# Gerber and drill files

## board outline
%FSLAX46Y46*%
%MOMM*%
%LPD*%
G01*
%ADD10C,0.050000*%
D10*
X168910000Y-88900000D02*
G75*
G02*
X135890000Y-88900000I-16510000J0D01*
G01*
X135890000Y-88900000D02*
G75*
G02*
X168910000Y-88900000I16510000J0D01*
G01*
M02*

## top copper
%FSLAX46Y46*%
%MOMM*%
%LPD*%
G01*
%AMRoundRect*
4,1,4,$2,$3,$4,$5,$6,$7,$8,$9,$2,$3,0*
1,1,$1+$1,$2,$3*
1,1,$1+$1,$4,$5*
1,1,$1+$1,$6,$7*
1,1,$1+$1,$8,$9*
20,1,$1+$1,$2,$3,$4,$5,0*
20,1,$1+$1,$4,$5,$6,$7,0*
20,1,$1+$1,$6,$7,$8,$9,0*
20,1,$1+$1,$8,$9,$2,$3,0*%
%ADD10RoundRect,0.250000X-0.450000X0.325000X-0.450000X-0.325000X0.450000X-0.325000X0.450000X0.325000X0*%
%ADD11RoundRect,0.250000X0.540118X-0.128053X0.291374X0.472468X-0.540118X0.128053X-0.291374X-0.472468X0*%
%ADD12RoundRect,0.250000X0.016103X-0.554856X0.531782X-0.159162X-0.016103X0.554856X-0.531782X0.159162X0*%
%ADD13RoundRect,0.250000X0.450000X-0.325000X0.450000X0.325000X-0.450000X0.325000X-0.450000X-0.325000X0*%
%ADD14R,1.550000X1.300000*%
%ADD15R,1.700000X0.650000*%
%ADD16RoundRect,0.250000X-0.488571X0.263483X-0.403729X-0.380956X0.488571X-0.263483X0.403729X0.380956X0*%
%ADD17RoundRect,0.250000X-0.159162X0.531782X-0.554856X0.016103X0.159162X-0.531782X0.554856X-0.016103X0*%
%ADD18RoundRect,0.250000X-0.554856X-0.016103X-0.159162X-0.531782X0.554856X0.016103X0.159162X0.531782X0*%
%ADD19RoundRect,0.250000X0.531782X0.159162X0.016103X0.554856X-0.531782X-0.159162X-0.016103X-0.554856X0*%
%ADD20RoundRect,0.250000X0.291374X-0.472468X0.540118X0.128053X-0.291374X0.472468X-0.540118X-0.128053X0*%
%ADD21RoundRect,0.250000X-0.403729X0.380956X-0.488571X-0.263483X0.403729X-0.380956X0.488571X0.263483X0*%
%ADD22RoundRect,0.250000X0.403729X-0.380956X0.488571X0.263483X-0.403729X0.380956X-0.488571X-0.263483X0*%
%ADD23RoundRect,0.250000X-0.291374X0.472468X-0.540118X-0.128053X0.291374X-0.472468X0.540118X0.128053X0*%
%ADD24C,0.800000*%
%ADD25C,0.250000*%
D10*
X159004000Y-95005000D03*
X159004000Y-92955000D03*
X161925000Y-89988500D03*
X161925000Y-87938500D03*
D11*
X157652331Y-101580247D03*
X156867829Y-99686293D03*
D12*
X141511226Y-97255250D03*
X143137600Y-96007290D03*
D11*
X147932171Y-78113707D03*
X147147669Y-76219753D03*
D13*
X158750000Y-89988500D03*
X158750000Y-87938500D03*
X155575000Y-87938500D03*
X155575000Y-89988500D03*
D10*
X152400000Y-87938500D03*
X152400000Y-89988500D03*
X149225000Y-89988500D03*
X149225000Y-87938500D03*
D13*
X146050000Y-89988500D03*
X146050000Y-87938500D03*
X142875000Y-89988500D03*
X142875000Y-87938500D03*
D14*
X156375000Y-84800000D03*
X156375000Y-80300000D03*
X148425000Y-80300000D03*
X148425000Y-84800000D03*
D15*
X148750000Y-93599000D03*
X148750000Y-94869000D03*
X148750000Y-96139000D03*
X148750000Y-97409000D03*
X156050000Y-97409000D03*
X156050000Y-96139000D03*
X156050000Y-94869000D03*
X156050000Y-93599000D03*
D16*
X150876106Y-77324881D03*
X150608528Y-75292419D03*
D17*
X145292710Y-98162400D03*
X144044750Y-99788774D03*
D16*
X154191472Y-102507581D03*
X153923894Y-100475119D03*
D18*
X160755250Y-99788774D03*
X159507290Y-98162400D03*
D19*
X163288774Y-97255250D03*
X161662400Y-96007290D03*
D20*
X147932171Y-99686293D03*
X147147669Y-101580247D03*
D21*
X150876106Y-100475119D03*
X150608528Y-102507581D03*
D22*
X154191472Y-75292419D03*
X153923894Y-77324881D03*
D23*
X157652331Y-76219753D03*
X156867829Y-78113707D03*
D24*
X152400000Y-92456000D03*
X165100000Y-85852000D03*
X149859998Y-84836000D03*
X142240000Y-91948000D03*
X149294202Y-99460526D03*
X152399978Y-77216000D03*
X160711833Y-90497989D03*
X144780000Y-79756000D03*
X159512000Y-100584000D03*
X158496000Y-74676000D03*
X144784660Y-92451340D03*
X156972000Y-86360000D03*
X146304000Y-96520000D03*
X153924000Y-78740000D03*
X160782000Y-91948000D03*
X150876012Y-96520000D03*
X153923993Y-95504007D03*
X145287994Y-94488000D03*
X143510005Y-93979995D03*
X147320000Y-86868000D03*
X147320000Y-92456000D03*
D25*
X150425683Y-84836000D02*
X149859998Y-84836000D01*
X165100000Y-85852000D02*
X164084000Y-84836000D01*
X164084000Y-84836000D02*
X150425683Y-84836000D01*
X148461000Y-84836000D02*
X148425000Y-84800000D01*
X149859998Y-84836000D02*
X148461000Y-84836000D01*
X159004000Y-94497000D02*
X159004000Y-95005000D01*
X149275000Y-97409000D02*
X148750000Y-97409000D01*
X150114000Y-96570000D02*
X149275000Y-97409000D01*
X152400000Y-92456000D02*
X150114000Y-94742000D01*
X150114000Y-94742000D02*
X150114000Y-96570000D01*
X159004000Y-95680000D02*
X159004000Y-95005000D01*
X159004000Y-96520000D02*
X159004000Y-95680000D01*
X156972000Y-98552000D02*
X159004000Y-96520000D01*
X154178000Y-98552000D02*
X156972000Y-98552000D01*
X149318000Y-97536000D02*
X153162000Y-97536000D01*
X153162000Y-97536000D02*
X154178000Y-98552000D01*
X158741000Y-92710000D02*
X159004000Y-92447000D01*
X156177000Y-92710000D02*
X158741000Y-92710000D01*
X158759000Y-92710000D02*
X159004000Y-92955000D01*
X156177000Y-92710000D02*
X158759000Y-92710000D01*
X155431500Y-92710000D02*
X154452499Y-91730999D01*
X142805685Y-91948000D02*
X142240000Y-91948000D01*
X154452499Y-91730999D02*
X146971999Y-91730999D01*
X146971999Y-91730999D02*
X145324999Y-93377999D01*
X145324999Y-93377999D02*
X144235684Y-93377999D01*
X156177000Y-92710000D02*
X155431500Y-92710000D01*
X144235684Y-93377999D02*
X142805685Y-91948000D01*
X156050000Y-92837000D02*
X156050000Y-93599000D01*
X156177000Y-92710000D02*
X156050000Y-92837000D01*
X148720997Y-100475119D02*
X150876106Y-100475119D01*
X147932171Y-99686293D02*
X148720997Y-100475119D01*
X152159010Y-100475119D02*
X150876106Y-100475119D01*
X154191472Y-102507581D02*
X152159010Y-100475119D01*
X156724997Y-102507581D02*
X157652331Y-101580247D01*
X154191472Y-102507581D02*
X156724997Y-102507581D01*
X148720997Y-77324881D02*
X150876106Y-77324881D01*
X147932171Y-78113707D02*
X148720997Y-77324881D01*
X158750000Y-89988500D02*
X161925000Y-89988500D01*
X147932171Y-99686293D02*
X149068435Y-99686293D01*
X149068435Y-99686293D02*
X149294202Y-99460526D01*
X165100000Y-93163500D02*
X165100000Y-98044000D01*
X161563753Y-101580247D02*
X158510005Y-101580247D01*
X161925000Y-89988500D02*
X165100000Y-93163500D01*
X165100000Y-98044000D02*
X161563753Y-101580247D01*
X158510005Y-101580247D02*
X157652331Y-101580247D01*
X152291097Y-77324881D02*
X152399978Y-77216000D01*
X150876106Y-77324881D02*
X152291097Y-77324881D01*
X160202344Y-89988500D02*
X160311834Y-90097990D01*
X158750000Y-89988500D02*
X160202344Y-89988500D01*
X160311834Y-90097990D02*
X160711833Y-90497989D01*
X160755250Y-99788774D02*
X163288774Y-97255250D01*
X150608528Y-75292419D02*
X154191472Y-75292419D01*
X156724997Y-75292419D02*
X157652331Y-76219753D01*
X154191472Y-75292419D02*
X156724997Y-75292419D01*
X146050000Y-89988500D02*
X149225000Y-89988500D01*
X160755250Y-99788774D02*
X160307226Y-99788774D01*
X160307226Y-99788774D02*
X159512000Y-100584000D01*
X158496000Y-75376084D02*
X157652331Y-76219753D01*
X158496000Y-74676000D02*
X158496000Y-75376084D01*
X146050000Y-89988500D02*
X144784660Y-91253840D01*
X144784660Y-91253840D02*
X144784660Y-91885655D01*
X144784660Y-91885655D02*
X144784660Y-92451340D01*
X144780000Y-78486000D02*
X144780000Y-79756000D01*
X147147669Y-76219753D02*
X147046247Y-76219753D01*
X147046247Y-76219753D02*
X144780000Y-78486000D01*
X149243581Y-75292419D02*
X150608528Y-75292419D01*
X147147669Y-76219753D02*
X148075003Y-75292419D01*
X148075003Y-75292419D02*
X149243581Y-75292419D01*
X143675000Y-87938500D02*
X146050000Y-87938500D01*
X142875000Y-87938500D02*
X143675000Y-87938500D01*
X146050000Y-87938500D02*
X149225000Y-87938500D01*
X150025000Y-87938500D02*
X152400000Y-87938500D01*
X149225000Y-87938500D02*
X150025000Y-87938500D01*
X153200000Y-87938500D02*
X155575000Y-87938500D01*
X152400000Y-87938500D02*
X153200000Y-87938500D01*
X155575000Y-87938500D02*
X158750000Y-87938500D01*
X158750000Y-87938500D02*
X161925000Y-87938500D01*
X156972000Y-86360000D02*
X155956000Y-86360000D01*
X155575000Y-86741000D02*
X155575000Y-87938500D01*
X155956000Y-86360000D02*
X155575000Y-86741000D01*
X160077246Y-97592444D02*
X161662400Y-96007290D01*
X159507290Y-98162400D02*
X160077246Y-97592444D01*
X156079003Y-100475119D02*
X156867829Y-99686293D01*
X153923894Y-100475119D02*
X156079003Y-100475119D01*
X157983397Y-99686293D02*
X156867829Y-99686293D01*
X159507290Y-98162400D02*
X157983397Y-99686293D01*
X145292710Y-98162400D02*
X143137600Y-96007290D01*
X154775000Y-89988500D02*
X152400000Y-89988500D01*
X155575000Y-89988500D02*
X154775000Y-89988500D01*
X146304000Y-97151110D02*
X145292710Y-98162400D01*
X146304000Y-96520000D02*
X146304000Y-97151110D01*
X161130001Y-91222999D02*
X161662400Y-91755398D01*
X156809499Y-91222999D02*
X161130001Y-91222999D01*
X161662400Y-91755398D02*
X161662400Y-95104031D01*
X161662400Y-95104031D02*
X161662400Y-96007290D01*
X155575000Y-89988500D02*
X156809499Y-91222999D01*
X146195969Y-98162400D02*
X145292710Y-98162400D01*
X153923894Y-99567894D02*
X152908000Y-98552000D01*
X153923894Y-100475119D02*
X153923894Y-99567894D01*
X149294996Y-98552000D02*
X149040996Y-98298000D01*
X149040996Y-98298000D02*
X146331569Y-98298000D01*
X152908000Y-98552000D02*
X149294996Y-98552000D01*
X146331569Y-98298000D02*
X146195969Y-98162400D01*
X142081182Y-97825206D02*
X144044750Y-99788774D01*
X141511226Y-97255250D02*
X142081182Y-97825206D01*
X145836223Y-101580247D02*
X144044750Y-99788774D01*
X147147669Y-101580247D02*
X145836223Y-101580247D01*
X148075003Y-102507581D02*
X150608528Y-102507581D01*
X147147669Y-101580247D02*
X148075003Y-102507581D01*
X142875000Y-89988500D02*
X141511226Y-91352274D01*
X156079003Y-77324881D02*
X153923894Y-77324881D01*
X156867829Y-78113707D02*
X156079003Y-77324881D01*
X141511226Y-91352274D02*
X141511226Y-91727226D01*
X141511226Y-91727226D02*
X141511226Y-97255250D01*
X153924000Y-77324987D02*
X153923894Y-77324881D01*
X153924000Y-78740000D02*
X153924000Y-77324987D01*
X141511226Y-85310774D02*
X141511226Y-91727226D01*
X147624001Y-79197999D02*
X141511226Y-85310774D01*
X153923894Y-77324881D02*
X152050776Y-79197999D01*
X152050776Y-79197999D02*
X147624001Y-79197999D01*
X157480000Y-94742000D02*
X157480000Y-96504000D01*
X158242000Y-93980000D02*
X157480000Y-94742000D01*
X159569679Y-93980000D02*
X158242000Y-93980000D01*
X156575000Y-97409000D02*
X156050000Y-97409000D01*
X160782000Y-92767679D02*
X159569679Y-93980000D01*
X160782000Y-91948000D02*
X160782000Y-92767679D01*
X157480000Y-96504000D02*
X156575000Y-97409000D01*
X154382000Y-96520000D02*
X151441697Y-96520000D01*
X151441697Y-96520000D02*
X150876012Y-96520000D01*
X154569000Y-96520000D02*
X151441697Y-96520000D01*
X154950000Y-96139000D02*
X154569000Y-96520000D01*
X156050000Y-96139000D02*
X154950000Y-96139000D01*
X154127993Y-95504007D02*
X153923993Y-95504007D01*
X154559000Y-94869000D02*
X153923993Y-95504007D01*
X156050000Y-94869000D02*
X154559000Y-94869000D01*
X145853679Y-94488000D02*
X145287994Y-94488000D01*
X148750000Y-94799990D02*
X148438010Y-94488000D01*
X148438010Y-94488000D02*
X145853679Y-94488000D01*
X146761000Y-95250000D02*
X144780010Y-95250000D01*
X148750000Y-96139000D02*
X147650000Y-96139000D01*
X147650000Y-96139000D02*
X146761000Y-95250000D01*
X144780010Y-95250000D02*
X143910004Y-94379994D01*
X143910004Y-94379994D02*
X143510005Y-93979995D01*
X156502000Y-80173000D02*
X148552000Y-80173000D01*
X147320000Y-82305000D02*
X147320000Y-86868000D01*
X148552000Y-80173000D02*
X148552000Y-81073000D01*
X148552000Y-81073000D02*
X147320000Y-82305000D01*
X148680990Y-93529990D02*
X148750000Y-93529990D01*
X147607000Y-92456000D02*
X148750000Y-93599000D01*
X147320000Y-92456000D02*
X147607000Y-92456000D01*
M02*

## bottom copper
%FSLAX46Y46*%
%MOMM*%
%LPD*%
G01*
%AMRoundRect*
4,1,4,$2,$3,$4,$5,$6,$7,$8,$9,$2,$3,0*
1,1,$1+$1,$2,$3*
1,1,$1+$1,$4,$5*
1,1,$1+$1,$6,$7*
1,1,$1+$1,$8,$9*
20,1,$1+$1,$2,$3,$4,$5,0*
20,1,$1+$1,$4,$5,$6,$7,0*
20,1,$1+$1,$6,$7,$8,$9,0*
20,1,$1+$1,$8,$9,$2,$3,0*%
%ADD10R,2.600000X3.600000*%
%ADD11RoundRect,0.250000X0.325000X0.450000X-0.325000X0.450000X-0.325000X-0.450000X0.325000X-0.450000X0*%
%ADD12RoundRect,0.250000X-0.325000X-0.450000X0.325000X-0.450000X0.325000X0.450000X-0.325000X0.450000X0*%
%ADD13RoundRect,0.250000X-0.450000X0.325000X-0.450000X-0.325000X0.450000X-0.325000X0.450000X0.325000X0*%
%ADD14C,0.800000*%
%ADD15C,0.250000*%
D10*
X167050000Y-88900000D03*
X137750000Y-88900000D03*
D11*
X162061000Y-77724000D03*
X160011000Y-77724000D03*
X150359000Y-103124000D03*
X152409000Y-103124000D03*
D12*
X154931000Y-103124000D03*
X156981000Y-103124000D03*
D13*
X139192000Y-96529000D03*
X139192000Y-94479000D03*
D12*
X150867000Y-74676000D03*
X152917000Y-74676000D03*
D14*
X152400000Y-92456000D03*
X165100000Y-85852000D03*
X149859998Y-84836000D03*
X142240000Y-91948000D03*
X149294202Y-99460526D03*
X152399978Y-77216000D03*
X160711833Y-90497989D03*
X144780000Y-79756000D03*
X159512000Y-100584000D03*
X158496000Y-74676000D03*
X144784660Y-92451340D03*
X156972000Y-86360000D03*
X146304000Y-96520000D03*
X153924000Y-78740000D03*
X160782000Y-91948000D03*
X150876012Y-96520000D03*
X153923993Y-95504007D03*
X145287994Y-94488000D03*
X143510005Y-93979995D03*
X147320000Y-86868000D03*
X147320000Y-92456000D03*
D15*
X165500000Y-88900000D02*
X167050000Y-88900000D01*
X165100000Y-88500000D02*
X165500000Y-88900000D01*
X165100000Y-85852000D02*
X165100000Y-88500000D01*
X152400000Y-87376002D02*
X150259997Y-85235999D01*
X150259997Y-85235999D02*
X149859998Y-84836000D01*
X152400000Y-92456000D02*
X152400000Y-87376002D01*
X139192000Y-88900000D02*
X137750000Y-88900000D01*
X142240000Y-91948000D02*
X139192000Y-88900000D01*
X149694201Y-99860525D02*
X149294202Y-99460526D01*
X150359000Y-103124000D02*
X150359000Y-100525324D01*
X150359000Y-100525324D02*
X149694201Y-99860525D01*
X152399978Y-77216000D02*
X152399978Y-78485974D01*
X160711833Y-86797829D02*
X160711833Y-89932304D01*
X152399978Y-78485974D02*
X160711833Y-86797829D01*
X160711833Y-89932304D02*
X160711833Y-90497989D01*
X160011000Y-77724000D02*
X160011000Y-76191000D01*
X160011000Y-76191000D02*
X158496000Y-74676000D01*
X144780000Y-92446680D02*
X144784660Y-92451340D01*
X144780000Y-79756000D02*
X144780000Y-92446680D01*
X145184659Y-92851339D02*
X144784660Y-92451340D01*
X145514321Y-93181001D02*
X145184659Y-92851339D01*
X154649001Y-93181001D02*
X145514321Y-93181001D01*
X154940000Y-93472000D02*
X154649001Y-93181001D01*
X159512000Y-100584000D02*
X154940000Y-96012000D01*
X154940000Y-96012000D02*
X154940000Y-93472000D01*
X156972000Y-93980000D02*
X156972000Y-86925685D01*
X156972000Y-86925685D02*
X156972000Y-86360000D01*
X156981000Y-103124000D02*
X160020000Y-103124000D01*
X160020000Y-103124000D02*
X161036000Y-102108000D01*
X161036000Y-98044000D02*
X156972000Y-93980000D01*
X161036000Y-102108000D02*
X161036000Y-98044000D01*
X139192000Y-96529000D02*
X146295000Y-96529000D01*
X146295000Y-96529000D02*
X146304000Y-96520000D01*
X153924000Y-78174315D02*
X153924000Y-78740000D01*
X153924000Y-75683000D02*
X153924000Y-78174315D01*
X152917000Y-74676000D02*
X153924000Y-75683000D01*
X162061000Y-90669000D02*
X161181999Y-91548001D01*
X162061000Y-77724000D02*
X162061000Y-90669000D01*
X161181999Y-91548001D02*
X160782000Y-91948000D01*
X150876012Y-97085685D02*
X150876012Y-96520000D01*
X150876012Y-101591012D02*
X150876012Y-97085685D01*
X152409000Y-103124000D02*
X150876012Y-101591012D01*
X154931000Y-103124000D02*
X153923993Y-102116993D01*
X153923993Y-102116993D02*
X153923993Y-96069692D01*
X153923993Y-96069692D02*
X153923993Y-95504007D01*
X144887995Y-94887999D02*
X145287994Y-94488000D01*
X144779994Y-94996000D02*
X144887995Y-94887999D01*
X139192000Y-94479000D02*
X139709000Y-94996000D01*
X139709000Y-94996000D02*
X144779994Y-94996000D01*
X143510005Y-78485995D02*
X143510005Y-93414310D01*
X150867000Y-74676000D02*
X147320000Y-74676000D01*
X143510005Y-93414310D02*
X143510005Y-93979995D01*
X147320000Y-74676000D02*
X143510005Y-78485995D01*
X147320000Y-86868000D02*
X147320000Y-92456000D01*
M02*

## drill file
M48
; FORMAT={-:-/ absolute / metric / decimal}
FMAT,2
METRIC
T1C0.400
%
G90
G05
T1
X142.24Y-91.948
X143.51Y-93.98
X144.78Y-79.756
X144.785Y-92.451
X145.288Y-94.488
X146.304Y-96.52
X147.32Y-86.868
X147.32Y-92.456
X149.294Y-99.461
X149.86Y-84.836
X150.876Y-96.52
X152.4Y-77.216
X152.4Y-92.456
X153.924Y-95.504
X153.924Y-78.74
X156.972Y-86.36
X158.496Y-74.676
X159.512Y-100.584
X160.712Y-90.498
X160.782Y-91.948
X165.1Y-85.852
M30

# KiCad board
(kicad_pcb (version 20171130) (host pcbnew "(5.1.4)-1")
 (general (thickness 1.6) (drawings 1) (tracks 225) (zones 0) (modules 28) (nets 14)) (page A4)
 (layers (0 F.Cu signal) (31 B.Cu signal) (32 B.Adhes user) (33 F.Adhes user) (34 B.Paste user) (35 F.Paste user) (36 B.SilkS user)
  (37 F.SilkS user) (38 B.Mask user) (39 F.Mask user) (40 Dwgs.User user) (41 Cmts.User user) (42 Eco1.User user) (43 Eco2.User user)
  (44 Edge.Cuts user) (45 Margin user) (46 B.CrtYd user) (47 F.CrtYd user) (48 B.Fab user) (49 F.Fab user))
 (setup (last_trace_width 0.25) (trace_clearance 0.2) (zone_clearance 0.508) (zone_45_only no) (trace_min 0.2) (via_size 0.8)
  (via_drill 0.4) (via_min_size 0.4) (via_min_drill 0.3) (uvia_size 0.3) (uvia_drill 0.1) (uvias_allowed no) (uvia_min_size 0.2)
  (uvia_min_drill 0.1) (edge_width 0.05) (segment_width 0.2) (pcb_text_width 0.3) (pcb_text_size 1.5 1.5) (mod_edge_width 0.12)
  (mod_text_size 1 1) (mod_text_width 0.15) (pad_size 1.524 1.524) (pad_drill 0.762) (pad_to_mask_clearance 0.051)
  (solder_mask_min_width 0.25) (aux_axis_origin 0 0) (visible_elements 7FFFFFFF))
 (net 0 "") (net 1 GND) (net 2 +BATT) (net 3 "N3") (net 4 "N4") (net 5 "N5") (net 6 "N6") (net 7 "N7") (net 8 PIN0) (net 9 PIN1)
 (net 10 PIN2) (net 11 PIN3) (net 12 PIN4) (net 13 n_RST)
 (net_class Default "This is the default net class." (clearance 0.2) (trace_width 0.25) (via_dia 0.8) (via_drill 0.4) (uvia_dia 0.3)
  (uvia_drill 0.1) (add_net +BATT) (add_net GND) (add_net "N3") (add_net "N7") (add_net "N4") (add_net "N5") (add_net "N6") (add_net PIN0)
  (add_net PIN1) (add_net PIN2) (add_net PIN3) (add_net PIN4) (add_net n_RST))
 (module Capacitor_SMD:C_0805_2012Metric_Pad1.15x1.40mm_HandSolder (layer F.Cu) (at 159.004 93.98 270)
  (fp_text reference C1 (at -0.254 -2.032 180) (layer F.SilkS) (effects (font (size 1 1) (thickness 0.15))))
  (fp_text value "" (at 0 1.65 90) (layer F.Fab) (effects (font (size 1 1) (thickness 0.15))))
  (pad 2 smd roundrect (at 1.025 0 270) (size 1.15 1.4) (layers F.Cu F.Paste F.Mask) (roundrect_rratio 0.217391) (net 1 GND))
  (pad 1 smd roundrect (at -1.025 0 270) (size 1.15 1.4) (layers F.Cu F.Paste F.Mask) (roundrect_rratio 0.217391) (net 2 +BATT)))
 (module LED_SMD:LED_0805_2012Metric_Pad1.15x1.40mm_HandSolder (layer F.Cu) (at 161.925 88.9635 270)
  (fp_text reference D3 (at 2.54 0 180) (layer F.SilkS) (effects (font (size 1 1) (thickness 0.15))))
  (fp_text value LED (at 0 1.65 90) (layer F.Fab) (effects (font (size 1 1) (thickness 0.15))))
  (pad 2 smd roundrect (at 1.025 0 270) (size 1.15 1.4) (layers F.Cu F.Paste F.Mask) (roundrect_rratio 0.217391) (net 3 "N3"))
  (pad 1 smd roundrect (at -1.025 0 270) (size 1.15 1.4) (layers F.Cu F.Paste F.Mask) (roundrect_rratio 0.217391) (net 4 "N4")))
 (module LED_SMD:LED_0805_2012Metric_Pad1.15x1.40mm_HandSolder (layer F.Cu) (at 157.26008 100.63327 112.5)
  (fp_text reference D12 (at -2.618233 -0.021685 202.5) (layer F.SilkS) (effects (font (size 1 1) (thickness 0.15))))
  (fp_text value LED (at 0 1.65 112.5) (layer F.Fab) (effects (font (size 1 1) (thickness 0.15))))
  (pad 1 smd roundrect (at -1.025 0 112.5) (size 1.15 1.4) (layers F.Cu F.Paste F.Mask) (roundrect_rratio 0.217391) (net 3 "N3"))
  (pad 2 smd roundrect (at 1.025 0 112.5) (size 1.15 1.4) (layers F.Cu F.Paste F.Mask) (roundrect_rratio 0.217391) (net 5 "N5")))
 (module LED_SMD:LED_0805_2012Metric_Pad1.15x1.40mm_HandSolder (layer F.Cu) (at 142.324413 96.63127 37.5)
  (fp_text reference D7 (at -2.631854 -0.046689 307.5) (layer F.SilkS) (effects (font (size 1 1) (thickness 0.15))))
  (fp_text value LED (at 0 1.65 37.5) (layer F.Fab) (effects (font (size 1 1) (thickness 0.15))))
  (pad 1 smd roundrect (at -1.025 0 37.5) (size 1.15 1.4) (layers F.Cu F.Paste F.Mask) (roundrect_rratio 0.217391) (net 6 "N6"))
  (pad 2 smd roundrect (at 1.025 0 37.5) (size 1.15 1.4) (layers F.Cu F.Paste F.Mask) (roundrect_rratio 0.217391) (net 5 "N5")))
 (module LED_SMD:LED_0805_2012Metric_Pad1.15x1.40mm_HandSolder (layer F.Cu) (at 147.53992 77.16673 112.5)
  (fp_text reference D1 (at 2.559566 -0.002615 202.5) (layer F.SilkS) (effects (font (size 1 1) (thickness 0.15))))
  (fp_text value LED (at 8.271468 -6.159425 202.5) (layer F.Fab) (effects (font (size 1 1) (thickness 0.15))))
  (pad 1 smd roundrect (at -1.025 0 112.5) (size 1.15 1.4) (layers F.Cu F.Paste F.Mask) (roundrect_rratio 0.217391) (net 3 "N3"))
  (pad 2 smd roundrect (at 1.025 0 112.5) (size 1.15 1.4) (layers F.Cu F.Paste F.Mask) (roundrect_rratio 0.217391) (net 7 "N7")))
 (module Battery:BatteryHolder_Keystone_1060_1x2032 (layer B.Cu) (at 152.4 88.9)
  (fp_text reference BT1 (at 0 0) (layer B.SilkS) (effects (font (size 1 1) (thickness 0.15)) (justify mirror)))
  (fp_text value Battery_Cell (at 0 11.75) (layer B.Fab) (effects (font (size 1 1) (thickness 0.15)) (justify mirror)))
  (pad 2 smd rect (at 14.65 0 180) (size 2.6 3.6) (layers B.Cu B.Paste B.Mask) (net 1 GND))
  (pad 1 smd rect (at -14.65 0 180) (size 2.6 3.6) (layers B.Cu B.Paste B.Mask) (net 2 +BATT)))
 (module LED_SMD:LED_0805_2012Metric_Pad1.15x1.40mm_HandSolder (layer F.Cu) (at 158.75 88.9635 90)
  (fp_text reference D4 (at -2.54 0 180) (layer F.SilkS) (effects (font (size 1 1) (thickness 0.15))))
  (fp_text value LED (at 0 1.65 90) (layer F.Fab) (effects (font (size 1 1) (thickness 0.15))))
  (pad 1 smd roundrect (at -1.025 0 90) (size 1.15 1.4) (layers F.Cu F.Paste F.Mask) (roundrect_rratio 0.217391) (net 3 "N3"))
  (pad 2 smd roundrect (at 1.025 0 90) (size 1.15 1.4) (layers F.Cu F.Paste F.Mask) (roundrect_rratio 0.217391) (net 4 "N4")))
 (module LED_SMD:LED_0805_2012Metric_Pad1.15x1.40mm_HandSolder (layer F.Cu) (at 155.575 88.9635 90)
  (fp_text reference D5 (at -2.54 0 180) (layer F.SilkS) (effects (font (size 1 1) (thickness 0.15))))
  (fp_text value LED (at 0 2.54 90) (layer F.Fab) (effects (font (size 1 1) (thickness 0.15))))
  (pad 2 smd roundrect (at 1.025 0 90) (size 1.15 1.4) (layers F.Cu F.Paste F.Mask) (roundrect_rratio 0.217391) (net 4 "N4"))
  (pad 1 smd roundrect (at -1.025 0 90) (size 1.15 1.4) (layers F.Cu F.Paste F.Mask) (roundrect_rratio 0.217391) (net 5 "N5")))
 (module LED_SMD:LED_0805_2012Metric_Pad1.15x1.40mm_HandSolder (layer F.Cu) (at 152.4 88.9635 270)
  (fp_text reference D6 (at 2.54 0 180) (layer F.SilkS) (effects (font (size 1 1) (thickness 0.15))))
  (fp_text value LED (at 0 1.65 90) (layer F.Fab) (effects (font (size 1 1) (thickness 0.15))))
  (pad 1 smd roundrect (at -1.025 0 270) (size 1.15 1.4) (layers F.Cu F.Paste F.Mask) (roundrect_rratio 0.217391) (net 4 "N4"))
  (pad 2 smd roundrect (at 1.025 0 270) (size 1.15 1.4) (layers F.Cu F.Paste F.Mask) (roundrect_rratio 0.217391) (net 5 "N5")))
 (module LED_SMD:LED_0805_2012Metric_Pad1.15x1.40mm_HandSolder (layer F.Cu) (at 149.225 88.9635 270)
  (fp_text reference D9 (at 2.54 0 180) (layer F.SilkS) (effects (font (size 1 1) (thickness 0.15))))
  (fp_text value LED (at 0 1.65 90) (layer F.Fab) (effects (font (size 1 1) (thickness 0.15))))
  (pad 2 smd roundrect (at 1.025 0 270) (size 1.15 1.4) (layers F.Cu F.Paste F.Mask) (roundrect_rratio 0.217391) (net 7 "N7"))
  (pad 1 smd roundrect (at -1.025 0 270) (size 1.15 1.4) (layers F.Cu F.Paste F.Mask) (roundrect_rratio 0.217391) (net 4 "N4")))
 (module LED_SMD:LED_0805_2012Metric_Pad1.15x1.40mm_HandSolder (layer F.Cu) (at 146.05 88.9635 90)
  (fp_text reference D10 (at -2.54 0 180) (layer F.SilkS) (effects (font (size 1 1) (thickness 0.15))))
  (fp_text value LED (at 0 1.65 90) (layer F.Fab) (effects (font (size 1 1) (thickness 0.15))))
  (pad 1 smd roundrect (at -1.025 0 90) (size 1.15 1.4) (layers F.Cu F.Paste F.Mask) (roundrect_rratio 0.217391) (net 7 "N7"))
  (pad 2 smd roundrect (at 1.025 0 90) (size 1.15 1.4) (layers F.Cu F.Paste F.Mask) (roundrect_rratio 0.217391) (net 4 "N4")))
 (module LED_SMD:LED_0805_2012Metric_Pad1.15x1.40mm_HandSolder (layer F.Cu) (at 142.875 88.9635 90)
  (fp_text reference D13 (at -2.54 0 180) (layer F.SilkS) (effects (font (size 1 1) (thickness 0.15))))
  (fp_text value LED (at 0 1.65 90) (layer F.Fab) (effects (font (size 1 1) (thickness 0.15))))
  (pad 1 smd roundrect (at -1.025 0 90) (size 1.15 1.4) (layers F.Cu F.Paste F.Mask) (roundrect_rratio 0.217391) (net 6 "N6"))
  (pad 2 smd roundrect (at 1.025 0 90) (size 1.15 1.4) (layers F.Cu F.Paste F.Mask) (roundrect_rratio 0.217391) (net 4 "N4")))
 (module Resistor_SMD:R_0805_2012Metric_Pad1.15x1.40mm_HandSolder (layer B.Cu) (at 161.036 77.724 180)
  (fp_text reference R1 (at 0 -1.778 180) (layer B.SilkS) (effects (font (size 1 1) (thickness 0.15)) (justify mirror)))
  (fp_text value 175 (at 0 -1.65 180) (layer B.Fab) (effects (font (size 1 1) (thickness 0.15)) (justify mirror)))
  (pad 1 smd roundrect (at -1.025 0 180) (size 1.15 1.4) (layers B.Cu B.Paste B.Mask) (roundrect_rratio 0.217391) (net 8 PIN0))
  (pad 2 smd roundrect (at 1.025 0 180) (size 1.15 1.4) (layers B.Cu B.Paste B.Mask) (roundrect_rratio 0.217391) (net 7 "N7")))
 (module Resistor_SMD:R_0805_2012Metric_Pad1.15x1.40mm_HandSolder (layer B.Cu) (at 151.384 103.124 180)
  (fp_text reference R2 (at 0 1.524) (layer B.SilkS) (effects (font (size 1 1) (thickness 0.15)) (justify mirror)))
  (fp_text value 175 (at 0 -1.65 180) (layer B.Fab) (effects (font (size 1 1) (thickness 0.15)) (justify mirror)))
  (pad 2 smd roundrect (at 1.025 0 180) (size 1.15 1.4) (layers B.Cu B.Paste B.Mask) (roundrect_rratio 0.217391) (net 3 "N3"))
  (pad 1 smd roundrect (at -1.025 0 180) (size 1.15 1.4) (layers B.Cu B.Paste B.Mask) (roundrect_rratio 0.217391) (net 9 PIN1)))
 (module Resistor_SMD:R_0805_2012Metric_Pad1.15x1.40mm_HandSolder (layer B.Cu) (at 155.956 103.124)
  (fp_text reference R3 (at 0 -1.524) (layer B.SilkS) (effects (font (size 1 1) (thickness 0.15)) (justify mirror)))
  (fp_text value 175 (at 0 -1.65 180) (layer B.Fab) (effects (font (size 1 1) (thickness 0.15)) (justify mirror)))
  (pad 1 smd roundrect (at -1.025 0) (size 1.15 1.4) (layers B.Cu B.Paste B.Mask) (roundrect_rratio 0.217391) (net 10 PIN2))
  (pad 2 smd roundrect (at 1.025 0) (size 1.15 1.4) (layers B.Cu B.Paste B.Mask) (roundrect_rratio 0.217391) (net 4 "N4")))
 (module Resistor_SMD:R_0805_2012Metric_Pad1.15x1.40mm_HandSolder (layer B.Cu) (at 139.192 95.504 270)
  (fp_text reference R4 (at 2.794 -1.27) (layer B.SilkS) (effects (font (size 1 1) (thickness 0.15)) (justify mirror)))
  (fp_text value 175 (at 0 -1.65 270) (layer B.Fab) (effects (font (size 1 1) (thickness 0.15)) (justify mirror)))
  (pad 2 smd roundrect (at 1.025 0 270) (size 1.15 1.4) (layers B.Cu B.Paste B.Mask) (roundrect_rratio 0.217391) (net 5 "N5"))
  (pad 1 smd roundrect (at -1.025 0 270) (size 1.15 1.4) (layers B.Cu B.Paste B.Mask) (roundrect_rratio 0.217391) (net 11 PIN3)))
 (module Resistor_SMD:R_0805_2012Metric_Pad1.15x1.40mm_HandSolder (layer B.Cu) (at 151.892 74.676)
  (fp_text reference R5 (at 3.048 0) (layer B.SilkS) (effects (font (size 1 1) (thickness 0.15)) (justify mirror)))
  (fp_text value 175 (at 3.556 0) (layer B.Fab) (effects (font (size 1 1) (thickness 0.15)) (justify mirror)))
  (pad 1 smd roundrect (at -1.025 0) (size 1.15 1.4) (layers B.Cu B.Paste B.Mask) (roundrect_rratio 0.217391) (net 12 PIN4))
  (pad 2 smd roundrect (at 1.025 0) (size 1.15 1.4) (layers B.Cu B.Paste B.Mask) (roundrect_rratio 0.217391) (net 6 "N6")))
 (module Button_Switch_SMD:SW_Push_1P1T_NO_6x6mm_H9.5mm (layer F.Cu) (at 152.4 82.55)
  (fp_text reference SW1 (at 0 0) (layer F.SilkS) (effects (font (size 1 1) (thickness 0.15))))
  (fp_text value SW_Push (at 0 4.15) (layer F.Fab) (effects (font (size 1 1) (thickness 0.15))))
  (pad 2 smd rect (at 3.975 2.25) (size 1.55 1.3) (layers F.Cu F.Paste F.Mask) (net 1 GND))
  (pad 1 smd rect (at 3.975 -2.25) (size 1.55 1.3) (layers F.Cu F.Paste F.Mask) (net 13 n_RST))
  (pad 1 smd rect (at -3.975 -2.25) (size 1.55 1.3) (layers F.Cu F.Paste F.Mask) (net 13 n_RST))
  (pad 2 smd rect (at -3.975 2.25) (size 1.55 1.3) (layers F.Cu F.Paste F.Mask) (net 1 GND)))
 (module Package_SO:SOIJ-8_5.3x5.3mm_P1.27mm (layer F.Cu) (at 152.4 95.504)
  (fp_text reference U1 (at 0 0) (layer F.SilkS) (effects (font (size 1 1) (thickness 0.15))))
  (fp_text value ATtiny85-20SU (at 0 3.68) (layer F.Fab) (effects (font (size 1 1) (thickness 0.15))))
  (pad 1 smd rect (at -3.65 -1.905) (size 1.7 0.65) (layers F.Cu F.Paste F.Mask) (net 13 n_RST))
  (pad 2 smd rect (at -3.65 -0.635) (size 1.7 0.65) (layers F.Cu F.Paste F.Mask) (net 11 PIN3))
  (pad 3 smd rect (at -3.65 0.635) (size 1.7 0.65) (layers F.Cu F.Paste F.Mask) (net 12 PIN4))
  (pad 4 smd rect (at -3.65 1.905) (size 1.7 0.65) (layers F.Cu F.Paste F.Mask) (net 1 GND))
  (pad 5 smd rect (at 3.65 1.905) (size 1.7 0.65) (layers F.Cu F.Paste F.Mask) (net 8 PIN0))
  (pad 6 smd rect (at 3.65 0.635) (size 1.7 0.65) (layers F.Cu F.Paste F.Mask) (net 9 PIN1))
  (pad 7 smd rect (at 3.65 -0.635) (size 1.7 0.65) (layers F.Cu F.Paste F.Mask) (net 10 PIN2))
  (pad 8 smd rect (at 3.65 -1.905) (size 1.7 0.65) (layers F.Cu F.Paste F.Mask) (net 2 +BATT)))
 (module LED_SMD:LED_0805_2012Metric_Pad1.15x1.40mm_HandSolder (layer F.Cu) (at 150.742317 76.30865 277.5)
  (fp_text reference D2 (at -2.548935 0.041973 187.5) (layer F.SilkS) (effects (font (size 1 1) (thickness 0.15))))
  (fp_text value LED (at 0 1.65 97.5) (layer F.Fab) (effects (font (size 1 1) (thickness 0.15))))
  (pad 2 smd roundrect (at 1.025 0 277.5) (size 1.15 1.4) (layers F.Cu F.Paste F.Mask) (roundrect_rratio 0.217391) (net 3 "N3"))
  (pad 1 smd roundrect (at -1.025 0 277.5) (size 1.15 1.4) (layers F.Cu F.Paste F.Mask) (roundrect_rratio 0.217391) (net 7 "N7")))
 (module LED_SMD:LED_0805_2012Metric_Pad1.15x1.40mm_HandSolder (layer F.Cu) (at 144.66873 98.975587 232.5)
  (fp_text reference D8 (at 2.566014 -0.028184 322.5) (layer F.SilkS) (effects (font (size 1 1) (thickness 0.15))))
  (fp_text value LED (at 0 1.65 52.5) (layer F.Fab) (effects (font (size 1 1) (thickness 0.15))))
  (pad 1 smd roundrect (at -1.025 0 232.5) (size 1.15 1.4) (layers F.Cu F.Paste F.Mask) (roundrect_rratio 0.217391) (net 5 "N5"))
  (pad 2 smd roundrect (at 1.025 0 232.5) (size 1.15 1.4) (layers F.Cu F.Paste F.Mask) (roundrect_rratio 0.217391) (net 6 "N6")))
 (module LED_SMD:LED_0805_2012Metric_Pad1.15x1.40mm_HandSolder (layer F.Cu) (at 154.057683 101.49135 277.5)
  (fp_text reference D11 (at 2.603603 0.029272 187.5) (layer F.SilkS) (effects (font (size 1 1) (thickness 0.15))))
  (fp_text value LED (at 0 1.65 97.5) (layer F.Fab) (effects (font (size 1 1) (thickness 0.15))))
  (pad 2 smd roundrect (at 1.025 0 277.5) (size 1.15 1.4) (layers F.Cu F.Paste F.Mask) (roundrect_rratio 0.217391) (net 3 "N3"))
  (pad 1 smd roundrect (at -1.025 0 277.5) (size 1.15 1.4) (layers F.Cu F.Paste F.Mask) (roundrect_rratio 0.217391) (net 5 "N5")))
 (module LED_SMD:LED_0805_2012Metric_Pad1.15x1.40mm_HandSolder (layer F.Cu) (at 160.13127 98.975587 307.5)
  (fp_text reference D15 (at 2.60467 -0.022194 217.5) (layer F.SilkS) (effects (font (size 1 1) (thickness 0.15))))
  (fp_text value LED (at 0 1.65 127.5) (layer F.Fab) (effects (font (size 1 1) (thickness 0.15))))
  (pad 2 smd roundrect (at 1.025 0 307.5) (size 1.15 1.4) (layers F.Cu F.Paste F.Mask) (roundrect_rratio 0.217391) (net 7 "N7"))
  (pad 1 smd roundrect (at -1.025 0 307.5) (size 1.15 1.4) (layers F.Cu F.Paste F.Mask) (roundrect_rratio 0.217391) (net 5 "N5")))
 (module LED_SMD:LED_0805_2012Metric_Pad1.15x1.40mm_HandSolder (layer F.Cu) (at 162.475587 96.63127 142.5)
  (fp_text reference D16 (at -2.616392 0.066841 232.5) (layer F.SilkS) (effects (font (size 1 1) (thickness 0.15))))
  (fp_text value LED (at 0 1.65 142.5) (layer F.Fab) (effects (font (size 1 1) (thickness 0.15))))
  (pad 1 smd roundrect (at -1.025 0 142.5) (size 1.15 1.4) (layers F.Cu F.Paste F.Mask) (roundrect_rratio 0.217391) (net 7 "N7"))
  (pad 2 smd roundrect (at 1.025 0 142.5) (size 1.15 1.4) (layers F.Cu F.Paste F.Mask) (roundrect_rratio 0.217391) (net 5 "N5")))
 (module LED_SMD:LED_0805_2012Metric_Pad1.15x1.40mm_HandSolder (layer F.Cu) (at 147.53992 100.63327 67.5)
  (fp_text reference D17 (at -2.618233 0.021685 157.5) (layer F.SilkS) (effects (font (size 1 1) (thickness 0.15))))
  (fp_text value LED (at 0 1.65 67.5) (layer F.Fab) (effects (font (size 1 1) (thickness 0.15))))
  (pad 2 smd roundrect (at 1.025 0 67.5) (size 1.15 1.4) (layers F.Cu F.Paste F.Mask) (roundrect_rratio 0.217391) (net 3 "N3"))
  (pad 1 smd roundrect (at -1.025 0 67.5) (size 1.15 1.4) (layers F.Cu F.Paste F.Mask) (roundrect_rratio 0.217391) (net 6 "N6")))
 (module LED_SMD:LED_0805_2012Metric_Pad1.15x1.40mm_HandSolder (layer F.Cu) (at 150.742317 101.49135 262.5)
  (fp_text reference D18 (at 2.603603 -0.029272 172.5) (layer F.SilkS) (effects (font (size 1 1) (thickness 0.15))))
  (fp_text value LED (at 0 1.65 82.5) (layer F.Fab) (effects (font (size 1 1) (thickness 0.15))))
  (pad 1 smd roundrect (at -1.025 0 262.5) (size 1.15 1.4) (layers F.Cu F.Paste F.Mask) (roundrect_rratio 0.217391) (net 3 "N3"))
  (pad 2 smd roundrect (at 1.025 0 262.5) (size 1.15 1.4) (layers F.Cu F.Paste F.Mask) (roundrect_rratio 0.217391) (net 6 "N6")))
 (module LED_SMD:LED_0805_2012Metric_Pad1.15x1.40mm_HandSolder (layer F.Cu) (at 154.057683 76.30865 82.5)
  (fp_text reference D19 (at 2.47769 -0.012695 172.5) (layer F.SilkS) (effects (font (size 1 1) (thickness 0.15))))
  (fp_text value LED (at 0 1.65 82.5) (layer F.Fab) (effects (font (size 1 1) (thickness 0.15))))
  (pad 2 smd roundrect (at 1.025 0 82.5) (size 1.15 1.4) (layers F.Cu F.Paste F.Mask) (roundrect_rratio 0.217391) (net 7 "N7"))
  (pad 1 smd roundrect (at -1.025 0 82.5) (size 1.15 1.4) (layers F.Cu F.Paste F.Mask) (roundrect_rratio 0.217391) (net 6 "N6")))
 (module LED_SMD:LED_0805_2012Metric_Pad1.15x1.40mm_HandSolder (layer F.Cu) (at 157.26008 77.16673 247.5)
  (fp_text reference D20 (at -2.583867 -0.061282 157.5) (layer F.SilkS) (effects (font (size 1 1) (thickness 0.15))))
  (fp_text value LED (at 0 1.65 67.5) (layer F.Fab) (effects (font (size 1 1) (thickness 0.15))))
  (pad 1 smd roundrect (at -1.025 0 247.5) (size 1.15 1.4) (layers F.Cu F.Paste F.Mask) (roundrect_rratio 0.217391) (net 7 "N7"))
  (pad 2 smd roundrect (at 1.025 0 247.5) (size 1.15 1.4) (layers F.Cu F.Paste F.Mask) (roundrect_rratio 0.217391) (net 6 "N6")))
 (gr_circle (center 152.4 88.9) (end 168.91 88.9) (layer Edge.Cuts) (width 0.05))
 (via (at 152.4 92.456) (size 0.8) (drill 0.4) (layers F.Cu B.Cu) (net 1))
 (via (at 165.1 85.852) (size 0.8) (drill 0.4) (layers F.Cu B.Cu) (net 1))
 (segment (start 165.5 88.9) (end 167.05 88.9) (width 0.25) (layer B.Cu) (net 1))
 (segment (start 165.1 88.5) (end 165.5 88.9) (width 0.25) (layer B.Cu) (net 1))
 (segment (start 165.1 85.852) (end 165.1 88.5) (width 0.25) (layer B.Cu) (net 1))
 (via (at 149.859998 84.836) (size 0.8) (drill 0.4) (layers F.Cu B.Cu) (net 1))
 (segment (start 152.4 87.376002) (end 150.259997 85.235999) (width 0.25) (layer B.Cu) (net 1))
 (segment (start 150.259997 85.235999) (end 149.859998 84.836) (width 0.25) (layer B.Cu) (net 1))
 (segment (start 152.4 92.456) (end 152.4 87.376002) (width 0.25) (layer B.Cu) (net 1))
 (segment (start 150.425683 84.836) (end 149.859998 84.836) (width 0.25) (layer F.Cu) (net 1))
 (segment (start 165.1 85.852) (end 164.084 84.836) (width 0.25) (layer F.Cu) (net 1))
 (segment (start 164.084 84.836) (end 150.425683 84.836) (width 0.25) (layer F.Cu) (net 1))
 (segment (start 148.461 84.836) (end 148.425 84.8) (width 0.25) (layer F.Cu) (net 1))
 (segment (start 149.859998 84.836) (end 148.461 84.836) (width 0.25) (layer F.Cu) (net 1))
 (segment (start 159.004 94.497) (end 159.004 95.005) (width 0.25) (layer F.Cu) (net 1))
 (segment (start 149.275 97.409) (end 148.75 97.409) (width 0.25) (layer F.Cu) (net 1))
 (segment (start 150.114 96.57) (end 149.275 97.409) (width 0.25) (layer F.Cu) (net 1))
 (segment (start 152.4 92.456) (end 150.114 94.742) (width 0.25) (layer F.Cu) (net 1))
 (segment (start 150.114 94.742) (end 150.114 96.57) (width 0.25) (layer F.Cu) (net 1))
 (segment (start 159.004 95.68) (end 159.004 95.005) (width 0.25) (layer F.Cu) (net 1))
 (segment (start 159.004 96.52) (end 159.004 95.68) (width 0.25) (layer F.Cu) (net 1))
 (segment (start 156.972 98.552) (end 159.004 96.52) (width 0.25) (layer F.Cu) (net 1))
 (segment (start 154.178 98.552) (end 156.972 98.552) (width 0.25) (layer F.Cu) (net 1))
 (segment (start 149.318 97.536) (end 153.162 97.536) (width 0.25) (layer F.Cu) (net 1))
 (segment (start 153.162 97.536) (end 154.178 98.552) (width 0.25) (layer F.Cu) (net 1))
 (via (at 142.24 91.948) (size 0.8) (drill 0.4) (layers F.Cu B.Cu) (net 2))
 (segment (start 139.192 88.9) (end 137.75 88.9) (width 0.25) (layer B.Cu) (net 2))
 (segment (start 142.24 91.948) (end 139.192 88.9) (width 0.25) (layer B.Cu) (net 2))
 (segment (start 158.741 92.71) (end 159.004 92.447) (width 0.25) (layer F.Cu) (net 2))
 (segment (start 156.177 92.71) (end 158.741 92.71) (width 0.25) (layer F.Cu) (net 2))
 (segment (start 158.759 92.71) (end 159.004 92.955) (width 0.25) (layer F.Cu) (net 2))
 (segment (start 156.177 92.71) (end 158.759 92.71) (width 0.25) (layer F.Cu) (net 2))
 (segment (start 155.4315 92.71) (end 154.452499 91.730999) (width 0.25) (layer F.Cu) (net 2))
 (segment (start 142.805685 91.948) (end 142.24 91.948) (width 0.25) (layer F.Cu) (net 2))
 (segment (start 154.452499 91.730999) (end 146.971999 91.730999) (width 0.25) (layer F.Cu) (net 2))
 (segment (start 146.971999 91.730999) (end 145.324999 93.377999) (width 0.25) (layer F.Cu) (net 2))
 (segment (start 145.324999 93.377999) (end 144.235684 93.377999) (width 0.25) (layer F.Cu) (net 2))
 (segment (start 156.177 92.71) (end 155.4315 92.71) (width 0.25) (layer F.Cu) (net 2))
 (segment (start 144.235684 93.377999) (end 142.805685 91.948) (width 0.25) (layer F.Cu) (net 2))
 (segment (start 156.05 92.837) (end 156.05 93.599) (width 0.25) (layer F.Cu) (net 2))
 (segment (start 156.177 92.71) (end 156.05 92.837) (width 0.25) (layer F.Cu) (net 2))
 (segment (start 148.720997 100.475119) (end 150.876106 100.475119) (width 0.25) (layer F.Cu) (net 3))
 (segment (start 147.932171 99.686293) (end 148.720997 100.475119) (width 0.25) (layer F.Cu) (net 3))
 (segment (start 152.15901 100.475119) (end 150.876106 100.475119) (width 0.25) (layer F.Cu) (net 3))
 (segment (start 154.191472 102.507581) (end 152.15901 100.475119) (width 0.25) (layer F.Cu) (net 3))
 (segment (start 156.724997 102.507581) (end 157.652331 101.580247) (width 0.25) (layer F.Cu) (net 3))
 (segment (start 154.191472 102.507581) (end 156.724997 102.507581) (width 0.25) (layer F.Cu) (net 3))
 (segment (start 148.720997 77.324881) (end 150.876106 77.324881) (width 0.25) (layer F.Cu) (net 3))
 (segment (start 147.932171 78.113707) (end 148.720997 77.324881) (width 0.25) (layer F.Cu) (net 3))
 (segment (start 158.75 89.9885) (end 161.925 89.9885) (width 0.25) (layer F.Cu) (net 3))
 (segment (start 149.694201 99.860525) (end 149.294202 99.460526) (width 0.25) (layer B.Cu) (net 3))
 (segment (start 150.359 103.124) (end 150.359 100.525324) (width 0.25) (layer B.Cu) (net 3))
 (segment (start 150.359 100.525324) (end 149.694201 99.860525) (width 0.25) (layer B.Cu) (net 3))
 (via (at 149.294202 99.460526) (size 0.8) (drill 0.4) (layers F.Cu B.Cu) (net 3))
 (segment (start 147.932171 99.686293) (end 149.068435 99.686293) (width 0.25) (layer F.Cu) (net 3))
 (segment (start 149.068435 99.686293) (end 149.294202 99.460526) (width 0.25) (layer F.Cu) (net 3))
 (segment (start 165.1 93.1635) (end 165.1 98.044) (width 0.25) (layer F.Cu) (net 3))
 (segment (start 161.563753 101.580247) (end 158.510005 101.580247) (width 0.25) (layer F.Cu) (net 3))
 (segment (start 161.925 89.9885) (end 165.1 93.1635) (width 0.25) (layer F.Cu) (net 3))
 (segment (start 165.1 98.044) (end 161.563753 101.580247) (width 0.25) (layer F.Cu) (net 3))
 (segment (start 158.510005 101.580247) (end 157.652331 101.580247) (width 0.25) (layer F.Cu) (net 3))
 (via (at 152.399978 77.216) (size 0.8) (drill 0.4) (layers F.Cu B.Cu) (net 3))
 (segment (start 152.291097 77.324881) (end 152.399978 77.216) (width 0.25) (layer F.Cu) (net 3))
 (segment (start 150.876106 77.324881) (end 152.291097 77.324881) (width 0.25) (layer F.Cu) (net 3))
 (segment (start 152.399978 77.216) (end 152.399978 78.485974) (width 0.25) (layer B.Cu) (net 3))
 (segment (start 160.711833 86.797829) (end 160.711833 89.932304) (width 0.25) (layer B.Cu) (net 3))
 (via (at 160.711833 90.497989) (size 0.8) (drill 0.4) (layers F.Cu B.Cu) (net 3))
 (segment (start 160.202344 89.9885) (end 160.311834 90.09799) (width 0.25) (layer F.Cu) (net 3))
 (segment (start 152.399978 78.485974) (end 160.711833 86.797829) (width 0.25) (layer B.Cu) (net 3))
 (segment (start 158.75 89.9885) (end 160.202344 89.9885) (width 0.25) (layer F.Cu) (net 3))
 (segment (start 160.311834 90.09799) (end 160.711833 90.497989) (width 0.25) (layer F.Cu) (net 3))
 (segment (start 160.711833 89.932304) (end 160.711833 90.497989) (width 0.25) (layer B.Cu) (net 3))
 (segment (start 160.75525 99.788774) (end 163.288774 97.25525) (width 0.25) (layer F.Cu) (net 7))
 (segment (start 150.608528 75.292419) (end 154.191472 75.292419) (width 0.25) (layer F.Cu) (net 7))
 (segment (start 156.724997 75.292419) (end 157.652331 76.219753) (width 0.25) (layer F.Cu) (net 7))
 (segment (start 154.191472 75.292419) (end 156.724997 75.292419) (width 0.25) (layer F.Cu) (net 7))
 (segment (start 146.05 89.9885) (end 149.225 89.9885) (width 0.25) (layer F.Cu) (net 7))
 (via (at 144.78 79.756) (size 0.8) (drill 0.4) (layers F.Cu B.Cu) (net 7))
 (via (at 159.512 100.584) (size 0.8) (drill 0.4) (layers F.Cu B.Cu) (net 7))
 (segment (start 160.75525 99.788774) (end 160.307226 99.788774) (width 0.25) (layer F.Cu) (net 7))
 (segment (start 160.307226 99.788774) (end 159.512 100.584) (width 0.25) (layer F.Cu) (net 7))
 (via (at 158.496 74.676) (size 0.8) (drill 0.4) (layers F.Cu B.Cu) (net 7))
 (segment (start 160.011 77.724) (end 160.011 76.191) (width 0.25) (layer B.Cu) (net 7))
 (segment (start 160.011 76.191) (end 158.496 74.676) (width 0.25) (layer B.Cu) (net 7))
 (segment (start 158.496 75.376084) (end 157.652331 76.219753) (width 0.25) (layer F.Cu) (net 7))
 (segment (start 158.496 74.676) (end 158.496 75.376084) (width 0.25) (layer F.Cu) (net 7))
 (segment (start 146.05 89.9885) (end 144.78466 91.25384) (width 0.25) (layer F.Cu) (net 7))
 (segment (start 144.78466 91.25384) (end 144.78466 91.885655) (width 0.25) (layer F.Cu) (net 7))
 (via (at 144.78466 92.45134) (size 0.8) (drill 0.4) (layers F.Cu B.Cu) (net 7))
 (segment (start 144.78 92.44668) (end 144.78466 92.45134) (width 0.25) (layer B.Cu) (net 7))
 (segment (start 144.78 79.756) (end 144.78 92.44668) (width 0.25) (layer B.Cu) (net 7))
 (segment (start 144.78466 91.885655) (end 144.78466 92.45134) (width 0.25) (layer F.Cu) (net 7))
 (segment (start 145.184659 92.851339) (end 144.78466 92.45134) (width 0.25) (layer B.Cu) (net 7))
 (segment (start 145.514321 93.181001) (end 145.184659 92.851339) (width 0.25) (layer B.Cu) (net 7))
 (segment (start 154.649001 93.181001) (end 145.514321 93.181001) (width 0.25) (layer B.Cu) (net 7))
 (segment (start 154.94 93.472) (end 154.649001 93.181001) (width 0.25) (layer B.Cu) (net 7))
 (segment (start 159.512 100.584) (end 154.94 96.012) (width 0.25) (layer B.Cu) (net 7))
 (segment (start 154.94 96.012) (end 154.94 93.472) (width 0.25) (layer B.Cu) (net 7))
 (segment (start 144.78 78.486) (end 144.78 79.756) (width 0.25) (layer F.Cu) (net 7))
 (segment (start 147.147669 76.219753) (end 147.046247 76.219753) (width 0.25) (layer F.Cu) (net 7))
 (segment (start 147.046247 76.219753) (end 144.78 78.486) (width 0.25) (layer F.Cu) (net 7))
 (segment (start 149.243581 75.292419) (end 150.608528 75.292419) (width 0.25) (layer F.Cu) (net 7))
 (segment (start 147.147669 76.219753) (end 148.075003 75.292419) (width 0.25) (layer F.Cu) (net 7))
 (segment (start 148.075003 75.292419) (end 149.243581 75.292419) (width 0.25) (layer F.Cu) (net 7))
 (segment (start 143.675 87.9385) (end 146.05 87.9385) (width 0.25) (layer F.Cu) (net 4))
 (segment (start 142.875 87.9385) (end 143.675 87.9385) (width 0.25) (layer F.Cu) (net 4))
 (segment (start 146.05 87.9385) (end 149.225 87.9385) (width 0.25) (layer F.Cu) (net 4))
 (segment (start 150.025 87.9385) (end 152.4 87.9385) (width 0.25) (layer F.Cu) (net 4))
 (segment (start 149.225 87.9385) (end 150.025 87.9385) (width 0.25) (layer F.Cu) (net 4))
 (segment (start 153.2 87.9385) (end 155.575 87.9385) (width 0.25) (layer F.Cu) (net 4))
 (segment (start 152.4 87.9385) (end 153.2 87.9385) (width 0.25) (layer F.Cu) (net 4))
 (segment (start 155.575 87.9385) (end 158.75 87.9385) (width 0.25) (layer F.Cu) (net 4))
 (segment (start 158.75 87.9385) (end 161.925 87.9385) (width 0.25) (layer F.Cu) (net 4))
 (via (at 156.972 86.36) (size 0.8) (drill 0.4) (layers F.Cu B.Cu) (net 4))
 (segment (start 156.972 86.36) (end 155.956 86.36) (width 0.25) (layer F.Cu) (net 4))
 (segment (start 155.575 86.741) (end 155.575 87.9385) (width 0.25) (layer F.Cu) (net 4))
 (segment (start 155.956 86.36) (end 155.575 86.741) (width 0.25) (layer F.Cu) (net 4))
 (segment (start 156.972 93.98) (end 156.972 86.925685) (width 0.25) (layer B.Cu) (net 4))
 (segment (start 156.972 86.925685) (end 156.972 86.36) (width 0.25) (layer B.Cu) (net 4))
 (segment (start 156.981 103.124) (end 160.02 103.124) (width 0.25) (layer B.Cu) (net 4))
 (segment (start 160.02 103.124) (end 161.036 102.108) (width 0.25) (layer B.Cu) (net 4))
 (segment (start 161.036 98.044) (end 156.972 93.98) (width 0.25) (layer B.Cu) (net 4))
 (segment (start 161.036 102.108) (end 161.036 98.044) (width 0.25) (layer B.Cu) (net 4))
 (segment (start 160.077246 97.592444) (end 161.6624 96.00729) (width 0.25) (layer F.Cu) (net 5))
 (segment (start 159.50729 98.1624) (end 160.077246 97.592444) (width 0.25) (layer F.Cu) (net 5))
 (segment (start 156.079003 100.475119) (end 156.867829 99.686293) (width 0.25) (layer F.Cu) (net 5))
 (segment (start 153.923894 100.475119) (end 156.079003 100.475119) (width 0.25) (layer F.Cu) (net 5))
 (segment (start 157.983397 99.686293) (end 156.867829 99.686293) (width 0.25) (layer F.Cu) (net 5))
 (segment (start 159.50729 98.1624) (end 157.983397 99.686293) (width 0.25) (layer F.Cu) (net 5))
 (segment (start 145.29271 98.1624) (end 143.1376 96.00729) (width 0.25) (layer F.Cu) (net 5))
 (segment (start 154.775 89.9885) (end 152.4 89.9885) (width 0.25) (layer F.Cu) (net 5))
 (segment (start 155.575 89.9885) (end 154.775 89.9885) (width 0.25) (layer F.Cu) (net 5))
 (via (at 146.304 96.52) (size 0.8) (drill 0.4) (layers F.Cu B.Cu) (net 5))
 (segment (start 139.192 96.529) (end 146.295 96.529) (width 0.25) (layer B.Cu) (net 5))
 (segment (start 146.295 96.529) (end 146.304 96.52) (width 0.25) (layer B.Cu) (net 5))
 (segment (start 146.304 97.15111) (end 145.29271 98.1624) (width 0.25) (layer F.Cu) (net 5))
 (segment (start 146.304 96.52) (end 146.304 97.15111) (width 0.25) (layer F.Cu) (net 5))
 (segment (start 161.130001 91.222999) (end 161.6624 91.755398) (width 0.25) (layer F.Cu) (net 5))
 (segment (start 156.809499 91.222999) (end 161.130001 91.222999) (width 0.25) (layer F.Cu) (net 5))
 (segment (start 161.6624 91.755398) (end 161.6624 95.104031) (width 0.25) (layer F.Cu) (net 5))
 (segment (start 161.6624 95.104031) (end 161.6624 96.00729) (width 0.25) (layer F.Cu) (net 5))
 (segment (start 155.575 89.9885) (end 156.809499 91.222999) (width 0.25) (layer F.Cu) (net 5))
 (segment (start 146.195969 98.1624) (end 145.29271 98.1624) (width 0.25) (layer F.Cu) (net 5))
 (segment (start 153.923894 99.567894) (end 152.908 98.552) (width 0.25) (layer F.Cu) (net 5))
 (segment (start 153.923894 100.475119) (end 153.923894 99.567894) (width 0.25) (layer F.Cu) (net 5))
 (segment (start 149.294996 98.552) (end 149.040996 98.298) (width 0.25) (layer F.Cu) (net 5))
 (segment (start 149.040996 98.298) (end 146.331569 98.298) (width 0.25) (layer F.Cu) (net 5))
 (segment (start 152.908 98.552) (end 149.294996 98.552) (width 0.25) (layer F.Cu) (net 5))
 (segment (start 146.331569 98.298) (end 146.195969 98.1624) (width 0.25) (layer F.Cu) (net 5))
 (segment (start 142.081182 97.825206) (end 144.04475 99.788774) (width 0.25) (layer F.Cu) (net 6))
 (segment (start 141.511226 97.25525) (end 142.081182 97.825206) (width 0.25) (layer F.Cu) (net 6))
 (segment (start 145.836223 101.580247) (end 144.04475 99.788774) (width 0.25) (layer F.Cu) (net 6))
 (segment (start 147.147669 101.580247) (end 145.836223 101.580247) (width 0.25) (layer F.Cu) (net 6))
 (segment (start 148.075003 102.507581) (end 150.608528 102.507581) (width 0.25) (layer F.Cu) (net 6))
 (segment (start 147.147669 101.580247) (end 148.075003 102.507581) (width 0.25) (layer F.Cu) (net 6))
 (segment (start 142.875 89.9885) (end 141.511226 91.352274) (width 0.25) (layer F.Cu) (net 6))
 (segment (start 156.079003 77.324881) (end 153.923894 77.324881) (width 0.25) (layer F.Cu) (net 6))
 (segment (start 156.867829 78.113707) (end 156.079003 77.324881) (width 0.25) (layer F.Cu) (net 6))
 (segment (start 141.511226 91.352274) (end 141.511226 91.727226) (width 0.25) (layer F.Cu) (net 6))
 (segment (start 141.511226 91.727226) (end 141.511226 97.25525) (width 0.25) (layer F.Cu) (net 6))
 (via (at 153.924 78.74) (size 0.8) (drill 0.4) (layers F.Cu B.Cu) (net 6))
 (segment (start 153.924 77.324987) (end 153.923894 77.324881) (width 0.25) (layer F.Cu) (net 6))
 (segment (start 153.924 78.74) (end 153.924 77.324987) (width 0.25) (layer F.Cu) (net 6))
 (segment (start 153.924 78.174315) (end 153.924 78.74) (width 0.25) (layer B.Cu) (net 6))
 (segment (start 153.924 75.683) (end 153.924 78.174315) (width 0.25) (layer B.Cu) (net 6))
 (segment (start 152.917 74.676) (end 153.924 75.683) (width 0.25) (layer B.Cu) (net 6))
 (segment (start 141.511226 85.310774) (end 141.511226 91.727226) (width 0.25) (layer F.Cu) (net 6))
 (segment (start 147.624001 79.197999) (end 141.511226 85.310774) (width 0.25) (layer F.Cu) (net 6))
 (segment (start 153.923894 77.324881) (end 152.050776 79.197999) (width 0.25) (layer F.Cu) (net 6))
 (segment (start 152.050776 79.197999) (end 147.624001 79.197999) (width 0.25) (layer F.Cu) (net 6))
 (segment (start 162.061 90.669) (end 161.181999 91.548001) (width 0.25) (layer B.Cu) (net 8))
 (via (at 160.782 91.948) (size 0.8) (drill 0.4) (layers F.Cu B.Cu) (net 8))
 (segment (start 162.061 77.724) (end 162.061 90.669) (width 0.25) (layer B.Cu) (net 8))
 (segment (start 161.181999 91.548001) (end 160.782 91.948) (width 0.25) (layer B.Cu) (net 8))
 (segment (start 157.48 94.742) (end 157.48 96.504) (width 0.25) (layer F.Cu) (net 8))
 (segment (start 158.242 93.98) (end 157.48 94.742) (width 0.25) (layer F.Cu) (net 8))
 (segment (start 159.569679 93.98) (end 158.242 93.98) (width 0.25) (layer F.Cu) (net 8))
 (segment (start 156.575 97.409) (end 156.05 97.409) (width 0.25) (layer F.Cu) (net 8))
 (segment (start 160.782 92.767679) (end 159.569679 93.98) (width 0.25) (layer F.Cu) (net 8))
 (segment (start 160.782 91.948) (end 160.782 92.767679) (width 0.25) (layer F.Cu) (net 8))
 (segment (start 157.48 96.504) (end 156.575 97.409) (width 0.25) (layer F.Cu) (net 8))
 (segment (start 150.876012 97.085685) (end 150.876012 96.52) (width 0.25) (layer B.Cu) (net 9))
 (segment (start 150.876012 101.591012) (end 150.876012 97.085685) (width 0.25) (layer B.Cu) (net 9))
 (via (at 150.876012 96.52) (size 0.8) (drill 0.4) (layers F.Cu B.Cu) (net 9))
 (segment (start 152.409 103.124) (end 150.876012 101.591012) (width 0.25) (layer B.Cu) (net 9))
 (segment (start 154.382 96.52) (end 151.441697 96.52) (width 0.25) (layer F.Cu) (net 9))
 (segment (start 151.441697 96.52) (end 150.876012 96.52) (width 0.25) (layer F.Cu) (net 9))
 (segment (start 154.569 96.52) (end 151.441697 96.52) (width 0.25) (layer F.Cu) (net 9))
 (segment (start 154.95 96.139) (end 154.569 96.52) (width 0.25) (layer F.Cu) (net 9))
 (segment (start 156.05 96.139) (end 154.95 96.139) (width 0.25) (layer F.Cu) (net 9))
 (segment (start 154.931 103.124) (end 153.923993 102.116993) (width 0.25) (layer B.Cu) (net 10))
 (segment (start 153.923993 102.116993) (end 153.923993 96.069692) (width 0.25) (layer B.Cu) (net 10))
 (segment (start 153.923993 96.069692) (end 153.923993 95.504007) (width 0.25) (layer B.Cu) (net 10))
 (segment (start 154.127993 95.504007) (end 153.923993 95.504007) (width 0.25) (layer F.Cu) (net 10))
 (via (at 153.923993 95.504007) (size 0.8) (drill 0.4) (layers F.Cu B.Cu) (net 10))
 (segment (start 154.559 94.869) (end 153.923993 95.504007) (width 0.25) (layer F.Cu) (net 10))
 (segment (start 156.05 94.869) (end 154.559 94.869) (width 0.25) (layer F.Cu) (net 10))
 (via (at 145.287994 94.488) (size 0.8) (drill 0.4) (layers F.Cu B.Cu) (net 11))
 (segment (start 144.887995 94.887999) (end 145.287994 94.488) (width 0.25) (layer B.Cu) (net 11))
 (segment (start 144.779994 94.996) (end 144.887995 94.887999) (width 0.25) (layer B.Cu) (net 11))
 (segment (start 139.192 94.479) (end 139.709 94.996) (width 0.25) (layer B.Cu) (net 11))
 (segment (start 139.709 94.996) (end 144.779994 94.996) (width 0.25) (layer B.Cu) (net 11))
 (segment (start 145.853679 94.488) (end 145.287994 94.488) (width 0.25) (layer F.Cu) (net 11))
 (segment (start 148.75 94.79999) (end 148.43801 94.488) (width 0.25) (layer F.Cu) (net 11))
 (segment (start 148.43801 94.488) (end 145.853679 94.488) (width 0.25) (layer F.Cu) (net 11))
 (segment (start 143.510005 78.485995) (end 143.510005 93.41431) (width 0.25) (layer B.Cu) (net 12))
 (segment (start 150.867 74.676) (end 147.32 74.676) (width 0.25) (layer B.Cu) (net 12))
 (segment (start 146.761 95.25) (end 144.78001 95.25) (width 0.25) (layer F.Cu) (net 12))
 (segment (start 143.510005 93.41431) (end 143.510005 93.979995) (width 0.25) (layer B.Cu) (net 12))
 (segment (start 148.75 96.139) (end 147.65 96.139) (width 0.25) (layer F.Cu) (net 12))
 (segment (start 147.65 96.139) (end 146.761 95.25) (width 0.25) (layer F.Cu) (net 12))
 (segment (start 144.78001 95.25) (end 143.910004 94.379994) (width 0.25) (layer F.Cu) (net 12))
 (segment (start 147.32 74.676) (end 143.510005 78.485995) (width 0.25) (layer B.Cu) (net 12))
 (via (at 143.510005 93.979995) (size 0.8) (drill 0.4) (layers F.Cu B.Cu) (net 12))
 (segment (start 143.910004 94.379994) (end 143.510005 93.979995) (width 0.25) (layer F.Cu) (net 12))
 (segment (start 156.502 80.173) (end 148.552 80.173) (width 0.25) (layer F.Cu) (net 13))
 (via (at 147.32 86.868) (size 0.8) (drill 0.4) (layers F.Cu B.Cu) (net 13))
 (segment (start 147.32 82.305) (end 147.32 86.868) (width 0.25) (layer F.Cu) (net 13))
 (segment (start 148.552 80.173) (end 148.552 81.073) (width 0.25) (layer F.Cu) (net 13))
 (segment (start 148.552 81.073) (end 147.32 82.305) (width 0.25) (layer F.Cu) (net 13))
 (segment (start 147.32 86.868) (end 147.32 92.456) (width 0.25) (layer B.Cu) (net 13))
 (via (at 147.32 92.456) (size 0.8) (drill 0.4) (layers F.Cu B.Cu) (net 13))
 (segment (start 148.68099 93.52999) (end 148.75 93.52999) (width 0.25) (layer F.Cu) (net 13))
 (segment (start 147.607 92.456) (end 148.75 93.599) (width 0.25) (layer F.Cu) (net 13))
 (segment (start 147.32 92.456) (end 147.607 92.456) (width 0.25) (layer F.Cu) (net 13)))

